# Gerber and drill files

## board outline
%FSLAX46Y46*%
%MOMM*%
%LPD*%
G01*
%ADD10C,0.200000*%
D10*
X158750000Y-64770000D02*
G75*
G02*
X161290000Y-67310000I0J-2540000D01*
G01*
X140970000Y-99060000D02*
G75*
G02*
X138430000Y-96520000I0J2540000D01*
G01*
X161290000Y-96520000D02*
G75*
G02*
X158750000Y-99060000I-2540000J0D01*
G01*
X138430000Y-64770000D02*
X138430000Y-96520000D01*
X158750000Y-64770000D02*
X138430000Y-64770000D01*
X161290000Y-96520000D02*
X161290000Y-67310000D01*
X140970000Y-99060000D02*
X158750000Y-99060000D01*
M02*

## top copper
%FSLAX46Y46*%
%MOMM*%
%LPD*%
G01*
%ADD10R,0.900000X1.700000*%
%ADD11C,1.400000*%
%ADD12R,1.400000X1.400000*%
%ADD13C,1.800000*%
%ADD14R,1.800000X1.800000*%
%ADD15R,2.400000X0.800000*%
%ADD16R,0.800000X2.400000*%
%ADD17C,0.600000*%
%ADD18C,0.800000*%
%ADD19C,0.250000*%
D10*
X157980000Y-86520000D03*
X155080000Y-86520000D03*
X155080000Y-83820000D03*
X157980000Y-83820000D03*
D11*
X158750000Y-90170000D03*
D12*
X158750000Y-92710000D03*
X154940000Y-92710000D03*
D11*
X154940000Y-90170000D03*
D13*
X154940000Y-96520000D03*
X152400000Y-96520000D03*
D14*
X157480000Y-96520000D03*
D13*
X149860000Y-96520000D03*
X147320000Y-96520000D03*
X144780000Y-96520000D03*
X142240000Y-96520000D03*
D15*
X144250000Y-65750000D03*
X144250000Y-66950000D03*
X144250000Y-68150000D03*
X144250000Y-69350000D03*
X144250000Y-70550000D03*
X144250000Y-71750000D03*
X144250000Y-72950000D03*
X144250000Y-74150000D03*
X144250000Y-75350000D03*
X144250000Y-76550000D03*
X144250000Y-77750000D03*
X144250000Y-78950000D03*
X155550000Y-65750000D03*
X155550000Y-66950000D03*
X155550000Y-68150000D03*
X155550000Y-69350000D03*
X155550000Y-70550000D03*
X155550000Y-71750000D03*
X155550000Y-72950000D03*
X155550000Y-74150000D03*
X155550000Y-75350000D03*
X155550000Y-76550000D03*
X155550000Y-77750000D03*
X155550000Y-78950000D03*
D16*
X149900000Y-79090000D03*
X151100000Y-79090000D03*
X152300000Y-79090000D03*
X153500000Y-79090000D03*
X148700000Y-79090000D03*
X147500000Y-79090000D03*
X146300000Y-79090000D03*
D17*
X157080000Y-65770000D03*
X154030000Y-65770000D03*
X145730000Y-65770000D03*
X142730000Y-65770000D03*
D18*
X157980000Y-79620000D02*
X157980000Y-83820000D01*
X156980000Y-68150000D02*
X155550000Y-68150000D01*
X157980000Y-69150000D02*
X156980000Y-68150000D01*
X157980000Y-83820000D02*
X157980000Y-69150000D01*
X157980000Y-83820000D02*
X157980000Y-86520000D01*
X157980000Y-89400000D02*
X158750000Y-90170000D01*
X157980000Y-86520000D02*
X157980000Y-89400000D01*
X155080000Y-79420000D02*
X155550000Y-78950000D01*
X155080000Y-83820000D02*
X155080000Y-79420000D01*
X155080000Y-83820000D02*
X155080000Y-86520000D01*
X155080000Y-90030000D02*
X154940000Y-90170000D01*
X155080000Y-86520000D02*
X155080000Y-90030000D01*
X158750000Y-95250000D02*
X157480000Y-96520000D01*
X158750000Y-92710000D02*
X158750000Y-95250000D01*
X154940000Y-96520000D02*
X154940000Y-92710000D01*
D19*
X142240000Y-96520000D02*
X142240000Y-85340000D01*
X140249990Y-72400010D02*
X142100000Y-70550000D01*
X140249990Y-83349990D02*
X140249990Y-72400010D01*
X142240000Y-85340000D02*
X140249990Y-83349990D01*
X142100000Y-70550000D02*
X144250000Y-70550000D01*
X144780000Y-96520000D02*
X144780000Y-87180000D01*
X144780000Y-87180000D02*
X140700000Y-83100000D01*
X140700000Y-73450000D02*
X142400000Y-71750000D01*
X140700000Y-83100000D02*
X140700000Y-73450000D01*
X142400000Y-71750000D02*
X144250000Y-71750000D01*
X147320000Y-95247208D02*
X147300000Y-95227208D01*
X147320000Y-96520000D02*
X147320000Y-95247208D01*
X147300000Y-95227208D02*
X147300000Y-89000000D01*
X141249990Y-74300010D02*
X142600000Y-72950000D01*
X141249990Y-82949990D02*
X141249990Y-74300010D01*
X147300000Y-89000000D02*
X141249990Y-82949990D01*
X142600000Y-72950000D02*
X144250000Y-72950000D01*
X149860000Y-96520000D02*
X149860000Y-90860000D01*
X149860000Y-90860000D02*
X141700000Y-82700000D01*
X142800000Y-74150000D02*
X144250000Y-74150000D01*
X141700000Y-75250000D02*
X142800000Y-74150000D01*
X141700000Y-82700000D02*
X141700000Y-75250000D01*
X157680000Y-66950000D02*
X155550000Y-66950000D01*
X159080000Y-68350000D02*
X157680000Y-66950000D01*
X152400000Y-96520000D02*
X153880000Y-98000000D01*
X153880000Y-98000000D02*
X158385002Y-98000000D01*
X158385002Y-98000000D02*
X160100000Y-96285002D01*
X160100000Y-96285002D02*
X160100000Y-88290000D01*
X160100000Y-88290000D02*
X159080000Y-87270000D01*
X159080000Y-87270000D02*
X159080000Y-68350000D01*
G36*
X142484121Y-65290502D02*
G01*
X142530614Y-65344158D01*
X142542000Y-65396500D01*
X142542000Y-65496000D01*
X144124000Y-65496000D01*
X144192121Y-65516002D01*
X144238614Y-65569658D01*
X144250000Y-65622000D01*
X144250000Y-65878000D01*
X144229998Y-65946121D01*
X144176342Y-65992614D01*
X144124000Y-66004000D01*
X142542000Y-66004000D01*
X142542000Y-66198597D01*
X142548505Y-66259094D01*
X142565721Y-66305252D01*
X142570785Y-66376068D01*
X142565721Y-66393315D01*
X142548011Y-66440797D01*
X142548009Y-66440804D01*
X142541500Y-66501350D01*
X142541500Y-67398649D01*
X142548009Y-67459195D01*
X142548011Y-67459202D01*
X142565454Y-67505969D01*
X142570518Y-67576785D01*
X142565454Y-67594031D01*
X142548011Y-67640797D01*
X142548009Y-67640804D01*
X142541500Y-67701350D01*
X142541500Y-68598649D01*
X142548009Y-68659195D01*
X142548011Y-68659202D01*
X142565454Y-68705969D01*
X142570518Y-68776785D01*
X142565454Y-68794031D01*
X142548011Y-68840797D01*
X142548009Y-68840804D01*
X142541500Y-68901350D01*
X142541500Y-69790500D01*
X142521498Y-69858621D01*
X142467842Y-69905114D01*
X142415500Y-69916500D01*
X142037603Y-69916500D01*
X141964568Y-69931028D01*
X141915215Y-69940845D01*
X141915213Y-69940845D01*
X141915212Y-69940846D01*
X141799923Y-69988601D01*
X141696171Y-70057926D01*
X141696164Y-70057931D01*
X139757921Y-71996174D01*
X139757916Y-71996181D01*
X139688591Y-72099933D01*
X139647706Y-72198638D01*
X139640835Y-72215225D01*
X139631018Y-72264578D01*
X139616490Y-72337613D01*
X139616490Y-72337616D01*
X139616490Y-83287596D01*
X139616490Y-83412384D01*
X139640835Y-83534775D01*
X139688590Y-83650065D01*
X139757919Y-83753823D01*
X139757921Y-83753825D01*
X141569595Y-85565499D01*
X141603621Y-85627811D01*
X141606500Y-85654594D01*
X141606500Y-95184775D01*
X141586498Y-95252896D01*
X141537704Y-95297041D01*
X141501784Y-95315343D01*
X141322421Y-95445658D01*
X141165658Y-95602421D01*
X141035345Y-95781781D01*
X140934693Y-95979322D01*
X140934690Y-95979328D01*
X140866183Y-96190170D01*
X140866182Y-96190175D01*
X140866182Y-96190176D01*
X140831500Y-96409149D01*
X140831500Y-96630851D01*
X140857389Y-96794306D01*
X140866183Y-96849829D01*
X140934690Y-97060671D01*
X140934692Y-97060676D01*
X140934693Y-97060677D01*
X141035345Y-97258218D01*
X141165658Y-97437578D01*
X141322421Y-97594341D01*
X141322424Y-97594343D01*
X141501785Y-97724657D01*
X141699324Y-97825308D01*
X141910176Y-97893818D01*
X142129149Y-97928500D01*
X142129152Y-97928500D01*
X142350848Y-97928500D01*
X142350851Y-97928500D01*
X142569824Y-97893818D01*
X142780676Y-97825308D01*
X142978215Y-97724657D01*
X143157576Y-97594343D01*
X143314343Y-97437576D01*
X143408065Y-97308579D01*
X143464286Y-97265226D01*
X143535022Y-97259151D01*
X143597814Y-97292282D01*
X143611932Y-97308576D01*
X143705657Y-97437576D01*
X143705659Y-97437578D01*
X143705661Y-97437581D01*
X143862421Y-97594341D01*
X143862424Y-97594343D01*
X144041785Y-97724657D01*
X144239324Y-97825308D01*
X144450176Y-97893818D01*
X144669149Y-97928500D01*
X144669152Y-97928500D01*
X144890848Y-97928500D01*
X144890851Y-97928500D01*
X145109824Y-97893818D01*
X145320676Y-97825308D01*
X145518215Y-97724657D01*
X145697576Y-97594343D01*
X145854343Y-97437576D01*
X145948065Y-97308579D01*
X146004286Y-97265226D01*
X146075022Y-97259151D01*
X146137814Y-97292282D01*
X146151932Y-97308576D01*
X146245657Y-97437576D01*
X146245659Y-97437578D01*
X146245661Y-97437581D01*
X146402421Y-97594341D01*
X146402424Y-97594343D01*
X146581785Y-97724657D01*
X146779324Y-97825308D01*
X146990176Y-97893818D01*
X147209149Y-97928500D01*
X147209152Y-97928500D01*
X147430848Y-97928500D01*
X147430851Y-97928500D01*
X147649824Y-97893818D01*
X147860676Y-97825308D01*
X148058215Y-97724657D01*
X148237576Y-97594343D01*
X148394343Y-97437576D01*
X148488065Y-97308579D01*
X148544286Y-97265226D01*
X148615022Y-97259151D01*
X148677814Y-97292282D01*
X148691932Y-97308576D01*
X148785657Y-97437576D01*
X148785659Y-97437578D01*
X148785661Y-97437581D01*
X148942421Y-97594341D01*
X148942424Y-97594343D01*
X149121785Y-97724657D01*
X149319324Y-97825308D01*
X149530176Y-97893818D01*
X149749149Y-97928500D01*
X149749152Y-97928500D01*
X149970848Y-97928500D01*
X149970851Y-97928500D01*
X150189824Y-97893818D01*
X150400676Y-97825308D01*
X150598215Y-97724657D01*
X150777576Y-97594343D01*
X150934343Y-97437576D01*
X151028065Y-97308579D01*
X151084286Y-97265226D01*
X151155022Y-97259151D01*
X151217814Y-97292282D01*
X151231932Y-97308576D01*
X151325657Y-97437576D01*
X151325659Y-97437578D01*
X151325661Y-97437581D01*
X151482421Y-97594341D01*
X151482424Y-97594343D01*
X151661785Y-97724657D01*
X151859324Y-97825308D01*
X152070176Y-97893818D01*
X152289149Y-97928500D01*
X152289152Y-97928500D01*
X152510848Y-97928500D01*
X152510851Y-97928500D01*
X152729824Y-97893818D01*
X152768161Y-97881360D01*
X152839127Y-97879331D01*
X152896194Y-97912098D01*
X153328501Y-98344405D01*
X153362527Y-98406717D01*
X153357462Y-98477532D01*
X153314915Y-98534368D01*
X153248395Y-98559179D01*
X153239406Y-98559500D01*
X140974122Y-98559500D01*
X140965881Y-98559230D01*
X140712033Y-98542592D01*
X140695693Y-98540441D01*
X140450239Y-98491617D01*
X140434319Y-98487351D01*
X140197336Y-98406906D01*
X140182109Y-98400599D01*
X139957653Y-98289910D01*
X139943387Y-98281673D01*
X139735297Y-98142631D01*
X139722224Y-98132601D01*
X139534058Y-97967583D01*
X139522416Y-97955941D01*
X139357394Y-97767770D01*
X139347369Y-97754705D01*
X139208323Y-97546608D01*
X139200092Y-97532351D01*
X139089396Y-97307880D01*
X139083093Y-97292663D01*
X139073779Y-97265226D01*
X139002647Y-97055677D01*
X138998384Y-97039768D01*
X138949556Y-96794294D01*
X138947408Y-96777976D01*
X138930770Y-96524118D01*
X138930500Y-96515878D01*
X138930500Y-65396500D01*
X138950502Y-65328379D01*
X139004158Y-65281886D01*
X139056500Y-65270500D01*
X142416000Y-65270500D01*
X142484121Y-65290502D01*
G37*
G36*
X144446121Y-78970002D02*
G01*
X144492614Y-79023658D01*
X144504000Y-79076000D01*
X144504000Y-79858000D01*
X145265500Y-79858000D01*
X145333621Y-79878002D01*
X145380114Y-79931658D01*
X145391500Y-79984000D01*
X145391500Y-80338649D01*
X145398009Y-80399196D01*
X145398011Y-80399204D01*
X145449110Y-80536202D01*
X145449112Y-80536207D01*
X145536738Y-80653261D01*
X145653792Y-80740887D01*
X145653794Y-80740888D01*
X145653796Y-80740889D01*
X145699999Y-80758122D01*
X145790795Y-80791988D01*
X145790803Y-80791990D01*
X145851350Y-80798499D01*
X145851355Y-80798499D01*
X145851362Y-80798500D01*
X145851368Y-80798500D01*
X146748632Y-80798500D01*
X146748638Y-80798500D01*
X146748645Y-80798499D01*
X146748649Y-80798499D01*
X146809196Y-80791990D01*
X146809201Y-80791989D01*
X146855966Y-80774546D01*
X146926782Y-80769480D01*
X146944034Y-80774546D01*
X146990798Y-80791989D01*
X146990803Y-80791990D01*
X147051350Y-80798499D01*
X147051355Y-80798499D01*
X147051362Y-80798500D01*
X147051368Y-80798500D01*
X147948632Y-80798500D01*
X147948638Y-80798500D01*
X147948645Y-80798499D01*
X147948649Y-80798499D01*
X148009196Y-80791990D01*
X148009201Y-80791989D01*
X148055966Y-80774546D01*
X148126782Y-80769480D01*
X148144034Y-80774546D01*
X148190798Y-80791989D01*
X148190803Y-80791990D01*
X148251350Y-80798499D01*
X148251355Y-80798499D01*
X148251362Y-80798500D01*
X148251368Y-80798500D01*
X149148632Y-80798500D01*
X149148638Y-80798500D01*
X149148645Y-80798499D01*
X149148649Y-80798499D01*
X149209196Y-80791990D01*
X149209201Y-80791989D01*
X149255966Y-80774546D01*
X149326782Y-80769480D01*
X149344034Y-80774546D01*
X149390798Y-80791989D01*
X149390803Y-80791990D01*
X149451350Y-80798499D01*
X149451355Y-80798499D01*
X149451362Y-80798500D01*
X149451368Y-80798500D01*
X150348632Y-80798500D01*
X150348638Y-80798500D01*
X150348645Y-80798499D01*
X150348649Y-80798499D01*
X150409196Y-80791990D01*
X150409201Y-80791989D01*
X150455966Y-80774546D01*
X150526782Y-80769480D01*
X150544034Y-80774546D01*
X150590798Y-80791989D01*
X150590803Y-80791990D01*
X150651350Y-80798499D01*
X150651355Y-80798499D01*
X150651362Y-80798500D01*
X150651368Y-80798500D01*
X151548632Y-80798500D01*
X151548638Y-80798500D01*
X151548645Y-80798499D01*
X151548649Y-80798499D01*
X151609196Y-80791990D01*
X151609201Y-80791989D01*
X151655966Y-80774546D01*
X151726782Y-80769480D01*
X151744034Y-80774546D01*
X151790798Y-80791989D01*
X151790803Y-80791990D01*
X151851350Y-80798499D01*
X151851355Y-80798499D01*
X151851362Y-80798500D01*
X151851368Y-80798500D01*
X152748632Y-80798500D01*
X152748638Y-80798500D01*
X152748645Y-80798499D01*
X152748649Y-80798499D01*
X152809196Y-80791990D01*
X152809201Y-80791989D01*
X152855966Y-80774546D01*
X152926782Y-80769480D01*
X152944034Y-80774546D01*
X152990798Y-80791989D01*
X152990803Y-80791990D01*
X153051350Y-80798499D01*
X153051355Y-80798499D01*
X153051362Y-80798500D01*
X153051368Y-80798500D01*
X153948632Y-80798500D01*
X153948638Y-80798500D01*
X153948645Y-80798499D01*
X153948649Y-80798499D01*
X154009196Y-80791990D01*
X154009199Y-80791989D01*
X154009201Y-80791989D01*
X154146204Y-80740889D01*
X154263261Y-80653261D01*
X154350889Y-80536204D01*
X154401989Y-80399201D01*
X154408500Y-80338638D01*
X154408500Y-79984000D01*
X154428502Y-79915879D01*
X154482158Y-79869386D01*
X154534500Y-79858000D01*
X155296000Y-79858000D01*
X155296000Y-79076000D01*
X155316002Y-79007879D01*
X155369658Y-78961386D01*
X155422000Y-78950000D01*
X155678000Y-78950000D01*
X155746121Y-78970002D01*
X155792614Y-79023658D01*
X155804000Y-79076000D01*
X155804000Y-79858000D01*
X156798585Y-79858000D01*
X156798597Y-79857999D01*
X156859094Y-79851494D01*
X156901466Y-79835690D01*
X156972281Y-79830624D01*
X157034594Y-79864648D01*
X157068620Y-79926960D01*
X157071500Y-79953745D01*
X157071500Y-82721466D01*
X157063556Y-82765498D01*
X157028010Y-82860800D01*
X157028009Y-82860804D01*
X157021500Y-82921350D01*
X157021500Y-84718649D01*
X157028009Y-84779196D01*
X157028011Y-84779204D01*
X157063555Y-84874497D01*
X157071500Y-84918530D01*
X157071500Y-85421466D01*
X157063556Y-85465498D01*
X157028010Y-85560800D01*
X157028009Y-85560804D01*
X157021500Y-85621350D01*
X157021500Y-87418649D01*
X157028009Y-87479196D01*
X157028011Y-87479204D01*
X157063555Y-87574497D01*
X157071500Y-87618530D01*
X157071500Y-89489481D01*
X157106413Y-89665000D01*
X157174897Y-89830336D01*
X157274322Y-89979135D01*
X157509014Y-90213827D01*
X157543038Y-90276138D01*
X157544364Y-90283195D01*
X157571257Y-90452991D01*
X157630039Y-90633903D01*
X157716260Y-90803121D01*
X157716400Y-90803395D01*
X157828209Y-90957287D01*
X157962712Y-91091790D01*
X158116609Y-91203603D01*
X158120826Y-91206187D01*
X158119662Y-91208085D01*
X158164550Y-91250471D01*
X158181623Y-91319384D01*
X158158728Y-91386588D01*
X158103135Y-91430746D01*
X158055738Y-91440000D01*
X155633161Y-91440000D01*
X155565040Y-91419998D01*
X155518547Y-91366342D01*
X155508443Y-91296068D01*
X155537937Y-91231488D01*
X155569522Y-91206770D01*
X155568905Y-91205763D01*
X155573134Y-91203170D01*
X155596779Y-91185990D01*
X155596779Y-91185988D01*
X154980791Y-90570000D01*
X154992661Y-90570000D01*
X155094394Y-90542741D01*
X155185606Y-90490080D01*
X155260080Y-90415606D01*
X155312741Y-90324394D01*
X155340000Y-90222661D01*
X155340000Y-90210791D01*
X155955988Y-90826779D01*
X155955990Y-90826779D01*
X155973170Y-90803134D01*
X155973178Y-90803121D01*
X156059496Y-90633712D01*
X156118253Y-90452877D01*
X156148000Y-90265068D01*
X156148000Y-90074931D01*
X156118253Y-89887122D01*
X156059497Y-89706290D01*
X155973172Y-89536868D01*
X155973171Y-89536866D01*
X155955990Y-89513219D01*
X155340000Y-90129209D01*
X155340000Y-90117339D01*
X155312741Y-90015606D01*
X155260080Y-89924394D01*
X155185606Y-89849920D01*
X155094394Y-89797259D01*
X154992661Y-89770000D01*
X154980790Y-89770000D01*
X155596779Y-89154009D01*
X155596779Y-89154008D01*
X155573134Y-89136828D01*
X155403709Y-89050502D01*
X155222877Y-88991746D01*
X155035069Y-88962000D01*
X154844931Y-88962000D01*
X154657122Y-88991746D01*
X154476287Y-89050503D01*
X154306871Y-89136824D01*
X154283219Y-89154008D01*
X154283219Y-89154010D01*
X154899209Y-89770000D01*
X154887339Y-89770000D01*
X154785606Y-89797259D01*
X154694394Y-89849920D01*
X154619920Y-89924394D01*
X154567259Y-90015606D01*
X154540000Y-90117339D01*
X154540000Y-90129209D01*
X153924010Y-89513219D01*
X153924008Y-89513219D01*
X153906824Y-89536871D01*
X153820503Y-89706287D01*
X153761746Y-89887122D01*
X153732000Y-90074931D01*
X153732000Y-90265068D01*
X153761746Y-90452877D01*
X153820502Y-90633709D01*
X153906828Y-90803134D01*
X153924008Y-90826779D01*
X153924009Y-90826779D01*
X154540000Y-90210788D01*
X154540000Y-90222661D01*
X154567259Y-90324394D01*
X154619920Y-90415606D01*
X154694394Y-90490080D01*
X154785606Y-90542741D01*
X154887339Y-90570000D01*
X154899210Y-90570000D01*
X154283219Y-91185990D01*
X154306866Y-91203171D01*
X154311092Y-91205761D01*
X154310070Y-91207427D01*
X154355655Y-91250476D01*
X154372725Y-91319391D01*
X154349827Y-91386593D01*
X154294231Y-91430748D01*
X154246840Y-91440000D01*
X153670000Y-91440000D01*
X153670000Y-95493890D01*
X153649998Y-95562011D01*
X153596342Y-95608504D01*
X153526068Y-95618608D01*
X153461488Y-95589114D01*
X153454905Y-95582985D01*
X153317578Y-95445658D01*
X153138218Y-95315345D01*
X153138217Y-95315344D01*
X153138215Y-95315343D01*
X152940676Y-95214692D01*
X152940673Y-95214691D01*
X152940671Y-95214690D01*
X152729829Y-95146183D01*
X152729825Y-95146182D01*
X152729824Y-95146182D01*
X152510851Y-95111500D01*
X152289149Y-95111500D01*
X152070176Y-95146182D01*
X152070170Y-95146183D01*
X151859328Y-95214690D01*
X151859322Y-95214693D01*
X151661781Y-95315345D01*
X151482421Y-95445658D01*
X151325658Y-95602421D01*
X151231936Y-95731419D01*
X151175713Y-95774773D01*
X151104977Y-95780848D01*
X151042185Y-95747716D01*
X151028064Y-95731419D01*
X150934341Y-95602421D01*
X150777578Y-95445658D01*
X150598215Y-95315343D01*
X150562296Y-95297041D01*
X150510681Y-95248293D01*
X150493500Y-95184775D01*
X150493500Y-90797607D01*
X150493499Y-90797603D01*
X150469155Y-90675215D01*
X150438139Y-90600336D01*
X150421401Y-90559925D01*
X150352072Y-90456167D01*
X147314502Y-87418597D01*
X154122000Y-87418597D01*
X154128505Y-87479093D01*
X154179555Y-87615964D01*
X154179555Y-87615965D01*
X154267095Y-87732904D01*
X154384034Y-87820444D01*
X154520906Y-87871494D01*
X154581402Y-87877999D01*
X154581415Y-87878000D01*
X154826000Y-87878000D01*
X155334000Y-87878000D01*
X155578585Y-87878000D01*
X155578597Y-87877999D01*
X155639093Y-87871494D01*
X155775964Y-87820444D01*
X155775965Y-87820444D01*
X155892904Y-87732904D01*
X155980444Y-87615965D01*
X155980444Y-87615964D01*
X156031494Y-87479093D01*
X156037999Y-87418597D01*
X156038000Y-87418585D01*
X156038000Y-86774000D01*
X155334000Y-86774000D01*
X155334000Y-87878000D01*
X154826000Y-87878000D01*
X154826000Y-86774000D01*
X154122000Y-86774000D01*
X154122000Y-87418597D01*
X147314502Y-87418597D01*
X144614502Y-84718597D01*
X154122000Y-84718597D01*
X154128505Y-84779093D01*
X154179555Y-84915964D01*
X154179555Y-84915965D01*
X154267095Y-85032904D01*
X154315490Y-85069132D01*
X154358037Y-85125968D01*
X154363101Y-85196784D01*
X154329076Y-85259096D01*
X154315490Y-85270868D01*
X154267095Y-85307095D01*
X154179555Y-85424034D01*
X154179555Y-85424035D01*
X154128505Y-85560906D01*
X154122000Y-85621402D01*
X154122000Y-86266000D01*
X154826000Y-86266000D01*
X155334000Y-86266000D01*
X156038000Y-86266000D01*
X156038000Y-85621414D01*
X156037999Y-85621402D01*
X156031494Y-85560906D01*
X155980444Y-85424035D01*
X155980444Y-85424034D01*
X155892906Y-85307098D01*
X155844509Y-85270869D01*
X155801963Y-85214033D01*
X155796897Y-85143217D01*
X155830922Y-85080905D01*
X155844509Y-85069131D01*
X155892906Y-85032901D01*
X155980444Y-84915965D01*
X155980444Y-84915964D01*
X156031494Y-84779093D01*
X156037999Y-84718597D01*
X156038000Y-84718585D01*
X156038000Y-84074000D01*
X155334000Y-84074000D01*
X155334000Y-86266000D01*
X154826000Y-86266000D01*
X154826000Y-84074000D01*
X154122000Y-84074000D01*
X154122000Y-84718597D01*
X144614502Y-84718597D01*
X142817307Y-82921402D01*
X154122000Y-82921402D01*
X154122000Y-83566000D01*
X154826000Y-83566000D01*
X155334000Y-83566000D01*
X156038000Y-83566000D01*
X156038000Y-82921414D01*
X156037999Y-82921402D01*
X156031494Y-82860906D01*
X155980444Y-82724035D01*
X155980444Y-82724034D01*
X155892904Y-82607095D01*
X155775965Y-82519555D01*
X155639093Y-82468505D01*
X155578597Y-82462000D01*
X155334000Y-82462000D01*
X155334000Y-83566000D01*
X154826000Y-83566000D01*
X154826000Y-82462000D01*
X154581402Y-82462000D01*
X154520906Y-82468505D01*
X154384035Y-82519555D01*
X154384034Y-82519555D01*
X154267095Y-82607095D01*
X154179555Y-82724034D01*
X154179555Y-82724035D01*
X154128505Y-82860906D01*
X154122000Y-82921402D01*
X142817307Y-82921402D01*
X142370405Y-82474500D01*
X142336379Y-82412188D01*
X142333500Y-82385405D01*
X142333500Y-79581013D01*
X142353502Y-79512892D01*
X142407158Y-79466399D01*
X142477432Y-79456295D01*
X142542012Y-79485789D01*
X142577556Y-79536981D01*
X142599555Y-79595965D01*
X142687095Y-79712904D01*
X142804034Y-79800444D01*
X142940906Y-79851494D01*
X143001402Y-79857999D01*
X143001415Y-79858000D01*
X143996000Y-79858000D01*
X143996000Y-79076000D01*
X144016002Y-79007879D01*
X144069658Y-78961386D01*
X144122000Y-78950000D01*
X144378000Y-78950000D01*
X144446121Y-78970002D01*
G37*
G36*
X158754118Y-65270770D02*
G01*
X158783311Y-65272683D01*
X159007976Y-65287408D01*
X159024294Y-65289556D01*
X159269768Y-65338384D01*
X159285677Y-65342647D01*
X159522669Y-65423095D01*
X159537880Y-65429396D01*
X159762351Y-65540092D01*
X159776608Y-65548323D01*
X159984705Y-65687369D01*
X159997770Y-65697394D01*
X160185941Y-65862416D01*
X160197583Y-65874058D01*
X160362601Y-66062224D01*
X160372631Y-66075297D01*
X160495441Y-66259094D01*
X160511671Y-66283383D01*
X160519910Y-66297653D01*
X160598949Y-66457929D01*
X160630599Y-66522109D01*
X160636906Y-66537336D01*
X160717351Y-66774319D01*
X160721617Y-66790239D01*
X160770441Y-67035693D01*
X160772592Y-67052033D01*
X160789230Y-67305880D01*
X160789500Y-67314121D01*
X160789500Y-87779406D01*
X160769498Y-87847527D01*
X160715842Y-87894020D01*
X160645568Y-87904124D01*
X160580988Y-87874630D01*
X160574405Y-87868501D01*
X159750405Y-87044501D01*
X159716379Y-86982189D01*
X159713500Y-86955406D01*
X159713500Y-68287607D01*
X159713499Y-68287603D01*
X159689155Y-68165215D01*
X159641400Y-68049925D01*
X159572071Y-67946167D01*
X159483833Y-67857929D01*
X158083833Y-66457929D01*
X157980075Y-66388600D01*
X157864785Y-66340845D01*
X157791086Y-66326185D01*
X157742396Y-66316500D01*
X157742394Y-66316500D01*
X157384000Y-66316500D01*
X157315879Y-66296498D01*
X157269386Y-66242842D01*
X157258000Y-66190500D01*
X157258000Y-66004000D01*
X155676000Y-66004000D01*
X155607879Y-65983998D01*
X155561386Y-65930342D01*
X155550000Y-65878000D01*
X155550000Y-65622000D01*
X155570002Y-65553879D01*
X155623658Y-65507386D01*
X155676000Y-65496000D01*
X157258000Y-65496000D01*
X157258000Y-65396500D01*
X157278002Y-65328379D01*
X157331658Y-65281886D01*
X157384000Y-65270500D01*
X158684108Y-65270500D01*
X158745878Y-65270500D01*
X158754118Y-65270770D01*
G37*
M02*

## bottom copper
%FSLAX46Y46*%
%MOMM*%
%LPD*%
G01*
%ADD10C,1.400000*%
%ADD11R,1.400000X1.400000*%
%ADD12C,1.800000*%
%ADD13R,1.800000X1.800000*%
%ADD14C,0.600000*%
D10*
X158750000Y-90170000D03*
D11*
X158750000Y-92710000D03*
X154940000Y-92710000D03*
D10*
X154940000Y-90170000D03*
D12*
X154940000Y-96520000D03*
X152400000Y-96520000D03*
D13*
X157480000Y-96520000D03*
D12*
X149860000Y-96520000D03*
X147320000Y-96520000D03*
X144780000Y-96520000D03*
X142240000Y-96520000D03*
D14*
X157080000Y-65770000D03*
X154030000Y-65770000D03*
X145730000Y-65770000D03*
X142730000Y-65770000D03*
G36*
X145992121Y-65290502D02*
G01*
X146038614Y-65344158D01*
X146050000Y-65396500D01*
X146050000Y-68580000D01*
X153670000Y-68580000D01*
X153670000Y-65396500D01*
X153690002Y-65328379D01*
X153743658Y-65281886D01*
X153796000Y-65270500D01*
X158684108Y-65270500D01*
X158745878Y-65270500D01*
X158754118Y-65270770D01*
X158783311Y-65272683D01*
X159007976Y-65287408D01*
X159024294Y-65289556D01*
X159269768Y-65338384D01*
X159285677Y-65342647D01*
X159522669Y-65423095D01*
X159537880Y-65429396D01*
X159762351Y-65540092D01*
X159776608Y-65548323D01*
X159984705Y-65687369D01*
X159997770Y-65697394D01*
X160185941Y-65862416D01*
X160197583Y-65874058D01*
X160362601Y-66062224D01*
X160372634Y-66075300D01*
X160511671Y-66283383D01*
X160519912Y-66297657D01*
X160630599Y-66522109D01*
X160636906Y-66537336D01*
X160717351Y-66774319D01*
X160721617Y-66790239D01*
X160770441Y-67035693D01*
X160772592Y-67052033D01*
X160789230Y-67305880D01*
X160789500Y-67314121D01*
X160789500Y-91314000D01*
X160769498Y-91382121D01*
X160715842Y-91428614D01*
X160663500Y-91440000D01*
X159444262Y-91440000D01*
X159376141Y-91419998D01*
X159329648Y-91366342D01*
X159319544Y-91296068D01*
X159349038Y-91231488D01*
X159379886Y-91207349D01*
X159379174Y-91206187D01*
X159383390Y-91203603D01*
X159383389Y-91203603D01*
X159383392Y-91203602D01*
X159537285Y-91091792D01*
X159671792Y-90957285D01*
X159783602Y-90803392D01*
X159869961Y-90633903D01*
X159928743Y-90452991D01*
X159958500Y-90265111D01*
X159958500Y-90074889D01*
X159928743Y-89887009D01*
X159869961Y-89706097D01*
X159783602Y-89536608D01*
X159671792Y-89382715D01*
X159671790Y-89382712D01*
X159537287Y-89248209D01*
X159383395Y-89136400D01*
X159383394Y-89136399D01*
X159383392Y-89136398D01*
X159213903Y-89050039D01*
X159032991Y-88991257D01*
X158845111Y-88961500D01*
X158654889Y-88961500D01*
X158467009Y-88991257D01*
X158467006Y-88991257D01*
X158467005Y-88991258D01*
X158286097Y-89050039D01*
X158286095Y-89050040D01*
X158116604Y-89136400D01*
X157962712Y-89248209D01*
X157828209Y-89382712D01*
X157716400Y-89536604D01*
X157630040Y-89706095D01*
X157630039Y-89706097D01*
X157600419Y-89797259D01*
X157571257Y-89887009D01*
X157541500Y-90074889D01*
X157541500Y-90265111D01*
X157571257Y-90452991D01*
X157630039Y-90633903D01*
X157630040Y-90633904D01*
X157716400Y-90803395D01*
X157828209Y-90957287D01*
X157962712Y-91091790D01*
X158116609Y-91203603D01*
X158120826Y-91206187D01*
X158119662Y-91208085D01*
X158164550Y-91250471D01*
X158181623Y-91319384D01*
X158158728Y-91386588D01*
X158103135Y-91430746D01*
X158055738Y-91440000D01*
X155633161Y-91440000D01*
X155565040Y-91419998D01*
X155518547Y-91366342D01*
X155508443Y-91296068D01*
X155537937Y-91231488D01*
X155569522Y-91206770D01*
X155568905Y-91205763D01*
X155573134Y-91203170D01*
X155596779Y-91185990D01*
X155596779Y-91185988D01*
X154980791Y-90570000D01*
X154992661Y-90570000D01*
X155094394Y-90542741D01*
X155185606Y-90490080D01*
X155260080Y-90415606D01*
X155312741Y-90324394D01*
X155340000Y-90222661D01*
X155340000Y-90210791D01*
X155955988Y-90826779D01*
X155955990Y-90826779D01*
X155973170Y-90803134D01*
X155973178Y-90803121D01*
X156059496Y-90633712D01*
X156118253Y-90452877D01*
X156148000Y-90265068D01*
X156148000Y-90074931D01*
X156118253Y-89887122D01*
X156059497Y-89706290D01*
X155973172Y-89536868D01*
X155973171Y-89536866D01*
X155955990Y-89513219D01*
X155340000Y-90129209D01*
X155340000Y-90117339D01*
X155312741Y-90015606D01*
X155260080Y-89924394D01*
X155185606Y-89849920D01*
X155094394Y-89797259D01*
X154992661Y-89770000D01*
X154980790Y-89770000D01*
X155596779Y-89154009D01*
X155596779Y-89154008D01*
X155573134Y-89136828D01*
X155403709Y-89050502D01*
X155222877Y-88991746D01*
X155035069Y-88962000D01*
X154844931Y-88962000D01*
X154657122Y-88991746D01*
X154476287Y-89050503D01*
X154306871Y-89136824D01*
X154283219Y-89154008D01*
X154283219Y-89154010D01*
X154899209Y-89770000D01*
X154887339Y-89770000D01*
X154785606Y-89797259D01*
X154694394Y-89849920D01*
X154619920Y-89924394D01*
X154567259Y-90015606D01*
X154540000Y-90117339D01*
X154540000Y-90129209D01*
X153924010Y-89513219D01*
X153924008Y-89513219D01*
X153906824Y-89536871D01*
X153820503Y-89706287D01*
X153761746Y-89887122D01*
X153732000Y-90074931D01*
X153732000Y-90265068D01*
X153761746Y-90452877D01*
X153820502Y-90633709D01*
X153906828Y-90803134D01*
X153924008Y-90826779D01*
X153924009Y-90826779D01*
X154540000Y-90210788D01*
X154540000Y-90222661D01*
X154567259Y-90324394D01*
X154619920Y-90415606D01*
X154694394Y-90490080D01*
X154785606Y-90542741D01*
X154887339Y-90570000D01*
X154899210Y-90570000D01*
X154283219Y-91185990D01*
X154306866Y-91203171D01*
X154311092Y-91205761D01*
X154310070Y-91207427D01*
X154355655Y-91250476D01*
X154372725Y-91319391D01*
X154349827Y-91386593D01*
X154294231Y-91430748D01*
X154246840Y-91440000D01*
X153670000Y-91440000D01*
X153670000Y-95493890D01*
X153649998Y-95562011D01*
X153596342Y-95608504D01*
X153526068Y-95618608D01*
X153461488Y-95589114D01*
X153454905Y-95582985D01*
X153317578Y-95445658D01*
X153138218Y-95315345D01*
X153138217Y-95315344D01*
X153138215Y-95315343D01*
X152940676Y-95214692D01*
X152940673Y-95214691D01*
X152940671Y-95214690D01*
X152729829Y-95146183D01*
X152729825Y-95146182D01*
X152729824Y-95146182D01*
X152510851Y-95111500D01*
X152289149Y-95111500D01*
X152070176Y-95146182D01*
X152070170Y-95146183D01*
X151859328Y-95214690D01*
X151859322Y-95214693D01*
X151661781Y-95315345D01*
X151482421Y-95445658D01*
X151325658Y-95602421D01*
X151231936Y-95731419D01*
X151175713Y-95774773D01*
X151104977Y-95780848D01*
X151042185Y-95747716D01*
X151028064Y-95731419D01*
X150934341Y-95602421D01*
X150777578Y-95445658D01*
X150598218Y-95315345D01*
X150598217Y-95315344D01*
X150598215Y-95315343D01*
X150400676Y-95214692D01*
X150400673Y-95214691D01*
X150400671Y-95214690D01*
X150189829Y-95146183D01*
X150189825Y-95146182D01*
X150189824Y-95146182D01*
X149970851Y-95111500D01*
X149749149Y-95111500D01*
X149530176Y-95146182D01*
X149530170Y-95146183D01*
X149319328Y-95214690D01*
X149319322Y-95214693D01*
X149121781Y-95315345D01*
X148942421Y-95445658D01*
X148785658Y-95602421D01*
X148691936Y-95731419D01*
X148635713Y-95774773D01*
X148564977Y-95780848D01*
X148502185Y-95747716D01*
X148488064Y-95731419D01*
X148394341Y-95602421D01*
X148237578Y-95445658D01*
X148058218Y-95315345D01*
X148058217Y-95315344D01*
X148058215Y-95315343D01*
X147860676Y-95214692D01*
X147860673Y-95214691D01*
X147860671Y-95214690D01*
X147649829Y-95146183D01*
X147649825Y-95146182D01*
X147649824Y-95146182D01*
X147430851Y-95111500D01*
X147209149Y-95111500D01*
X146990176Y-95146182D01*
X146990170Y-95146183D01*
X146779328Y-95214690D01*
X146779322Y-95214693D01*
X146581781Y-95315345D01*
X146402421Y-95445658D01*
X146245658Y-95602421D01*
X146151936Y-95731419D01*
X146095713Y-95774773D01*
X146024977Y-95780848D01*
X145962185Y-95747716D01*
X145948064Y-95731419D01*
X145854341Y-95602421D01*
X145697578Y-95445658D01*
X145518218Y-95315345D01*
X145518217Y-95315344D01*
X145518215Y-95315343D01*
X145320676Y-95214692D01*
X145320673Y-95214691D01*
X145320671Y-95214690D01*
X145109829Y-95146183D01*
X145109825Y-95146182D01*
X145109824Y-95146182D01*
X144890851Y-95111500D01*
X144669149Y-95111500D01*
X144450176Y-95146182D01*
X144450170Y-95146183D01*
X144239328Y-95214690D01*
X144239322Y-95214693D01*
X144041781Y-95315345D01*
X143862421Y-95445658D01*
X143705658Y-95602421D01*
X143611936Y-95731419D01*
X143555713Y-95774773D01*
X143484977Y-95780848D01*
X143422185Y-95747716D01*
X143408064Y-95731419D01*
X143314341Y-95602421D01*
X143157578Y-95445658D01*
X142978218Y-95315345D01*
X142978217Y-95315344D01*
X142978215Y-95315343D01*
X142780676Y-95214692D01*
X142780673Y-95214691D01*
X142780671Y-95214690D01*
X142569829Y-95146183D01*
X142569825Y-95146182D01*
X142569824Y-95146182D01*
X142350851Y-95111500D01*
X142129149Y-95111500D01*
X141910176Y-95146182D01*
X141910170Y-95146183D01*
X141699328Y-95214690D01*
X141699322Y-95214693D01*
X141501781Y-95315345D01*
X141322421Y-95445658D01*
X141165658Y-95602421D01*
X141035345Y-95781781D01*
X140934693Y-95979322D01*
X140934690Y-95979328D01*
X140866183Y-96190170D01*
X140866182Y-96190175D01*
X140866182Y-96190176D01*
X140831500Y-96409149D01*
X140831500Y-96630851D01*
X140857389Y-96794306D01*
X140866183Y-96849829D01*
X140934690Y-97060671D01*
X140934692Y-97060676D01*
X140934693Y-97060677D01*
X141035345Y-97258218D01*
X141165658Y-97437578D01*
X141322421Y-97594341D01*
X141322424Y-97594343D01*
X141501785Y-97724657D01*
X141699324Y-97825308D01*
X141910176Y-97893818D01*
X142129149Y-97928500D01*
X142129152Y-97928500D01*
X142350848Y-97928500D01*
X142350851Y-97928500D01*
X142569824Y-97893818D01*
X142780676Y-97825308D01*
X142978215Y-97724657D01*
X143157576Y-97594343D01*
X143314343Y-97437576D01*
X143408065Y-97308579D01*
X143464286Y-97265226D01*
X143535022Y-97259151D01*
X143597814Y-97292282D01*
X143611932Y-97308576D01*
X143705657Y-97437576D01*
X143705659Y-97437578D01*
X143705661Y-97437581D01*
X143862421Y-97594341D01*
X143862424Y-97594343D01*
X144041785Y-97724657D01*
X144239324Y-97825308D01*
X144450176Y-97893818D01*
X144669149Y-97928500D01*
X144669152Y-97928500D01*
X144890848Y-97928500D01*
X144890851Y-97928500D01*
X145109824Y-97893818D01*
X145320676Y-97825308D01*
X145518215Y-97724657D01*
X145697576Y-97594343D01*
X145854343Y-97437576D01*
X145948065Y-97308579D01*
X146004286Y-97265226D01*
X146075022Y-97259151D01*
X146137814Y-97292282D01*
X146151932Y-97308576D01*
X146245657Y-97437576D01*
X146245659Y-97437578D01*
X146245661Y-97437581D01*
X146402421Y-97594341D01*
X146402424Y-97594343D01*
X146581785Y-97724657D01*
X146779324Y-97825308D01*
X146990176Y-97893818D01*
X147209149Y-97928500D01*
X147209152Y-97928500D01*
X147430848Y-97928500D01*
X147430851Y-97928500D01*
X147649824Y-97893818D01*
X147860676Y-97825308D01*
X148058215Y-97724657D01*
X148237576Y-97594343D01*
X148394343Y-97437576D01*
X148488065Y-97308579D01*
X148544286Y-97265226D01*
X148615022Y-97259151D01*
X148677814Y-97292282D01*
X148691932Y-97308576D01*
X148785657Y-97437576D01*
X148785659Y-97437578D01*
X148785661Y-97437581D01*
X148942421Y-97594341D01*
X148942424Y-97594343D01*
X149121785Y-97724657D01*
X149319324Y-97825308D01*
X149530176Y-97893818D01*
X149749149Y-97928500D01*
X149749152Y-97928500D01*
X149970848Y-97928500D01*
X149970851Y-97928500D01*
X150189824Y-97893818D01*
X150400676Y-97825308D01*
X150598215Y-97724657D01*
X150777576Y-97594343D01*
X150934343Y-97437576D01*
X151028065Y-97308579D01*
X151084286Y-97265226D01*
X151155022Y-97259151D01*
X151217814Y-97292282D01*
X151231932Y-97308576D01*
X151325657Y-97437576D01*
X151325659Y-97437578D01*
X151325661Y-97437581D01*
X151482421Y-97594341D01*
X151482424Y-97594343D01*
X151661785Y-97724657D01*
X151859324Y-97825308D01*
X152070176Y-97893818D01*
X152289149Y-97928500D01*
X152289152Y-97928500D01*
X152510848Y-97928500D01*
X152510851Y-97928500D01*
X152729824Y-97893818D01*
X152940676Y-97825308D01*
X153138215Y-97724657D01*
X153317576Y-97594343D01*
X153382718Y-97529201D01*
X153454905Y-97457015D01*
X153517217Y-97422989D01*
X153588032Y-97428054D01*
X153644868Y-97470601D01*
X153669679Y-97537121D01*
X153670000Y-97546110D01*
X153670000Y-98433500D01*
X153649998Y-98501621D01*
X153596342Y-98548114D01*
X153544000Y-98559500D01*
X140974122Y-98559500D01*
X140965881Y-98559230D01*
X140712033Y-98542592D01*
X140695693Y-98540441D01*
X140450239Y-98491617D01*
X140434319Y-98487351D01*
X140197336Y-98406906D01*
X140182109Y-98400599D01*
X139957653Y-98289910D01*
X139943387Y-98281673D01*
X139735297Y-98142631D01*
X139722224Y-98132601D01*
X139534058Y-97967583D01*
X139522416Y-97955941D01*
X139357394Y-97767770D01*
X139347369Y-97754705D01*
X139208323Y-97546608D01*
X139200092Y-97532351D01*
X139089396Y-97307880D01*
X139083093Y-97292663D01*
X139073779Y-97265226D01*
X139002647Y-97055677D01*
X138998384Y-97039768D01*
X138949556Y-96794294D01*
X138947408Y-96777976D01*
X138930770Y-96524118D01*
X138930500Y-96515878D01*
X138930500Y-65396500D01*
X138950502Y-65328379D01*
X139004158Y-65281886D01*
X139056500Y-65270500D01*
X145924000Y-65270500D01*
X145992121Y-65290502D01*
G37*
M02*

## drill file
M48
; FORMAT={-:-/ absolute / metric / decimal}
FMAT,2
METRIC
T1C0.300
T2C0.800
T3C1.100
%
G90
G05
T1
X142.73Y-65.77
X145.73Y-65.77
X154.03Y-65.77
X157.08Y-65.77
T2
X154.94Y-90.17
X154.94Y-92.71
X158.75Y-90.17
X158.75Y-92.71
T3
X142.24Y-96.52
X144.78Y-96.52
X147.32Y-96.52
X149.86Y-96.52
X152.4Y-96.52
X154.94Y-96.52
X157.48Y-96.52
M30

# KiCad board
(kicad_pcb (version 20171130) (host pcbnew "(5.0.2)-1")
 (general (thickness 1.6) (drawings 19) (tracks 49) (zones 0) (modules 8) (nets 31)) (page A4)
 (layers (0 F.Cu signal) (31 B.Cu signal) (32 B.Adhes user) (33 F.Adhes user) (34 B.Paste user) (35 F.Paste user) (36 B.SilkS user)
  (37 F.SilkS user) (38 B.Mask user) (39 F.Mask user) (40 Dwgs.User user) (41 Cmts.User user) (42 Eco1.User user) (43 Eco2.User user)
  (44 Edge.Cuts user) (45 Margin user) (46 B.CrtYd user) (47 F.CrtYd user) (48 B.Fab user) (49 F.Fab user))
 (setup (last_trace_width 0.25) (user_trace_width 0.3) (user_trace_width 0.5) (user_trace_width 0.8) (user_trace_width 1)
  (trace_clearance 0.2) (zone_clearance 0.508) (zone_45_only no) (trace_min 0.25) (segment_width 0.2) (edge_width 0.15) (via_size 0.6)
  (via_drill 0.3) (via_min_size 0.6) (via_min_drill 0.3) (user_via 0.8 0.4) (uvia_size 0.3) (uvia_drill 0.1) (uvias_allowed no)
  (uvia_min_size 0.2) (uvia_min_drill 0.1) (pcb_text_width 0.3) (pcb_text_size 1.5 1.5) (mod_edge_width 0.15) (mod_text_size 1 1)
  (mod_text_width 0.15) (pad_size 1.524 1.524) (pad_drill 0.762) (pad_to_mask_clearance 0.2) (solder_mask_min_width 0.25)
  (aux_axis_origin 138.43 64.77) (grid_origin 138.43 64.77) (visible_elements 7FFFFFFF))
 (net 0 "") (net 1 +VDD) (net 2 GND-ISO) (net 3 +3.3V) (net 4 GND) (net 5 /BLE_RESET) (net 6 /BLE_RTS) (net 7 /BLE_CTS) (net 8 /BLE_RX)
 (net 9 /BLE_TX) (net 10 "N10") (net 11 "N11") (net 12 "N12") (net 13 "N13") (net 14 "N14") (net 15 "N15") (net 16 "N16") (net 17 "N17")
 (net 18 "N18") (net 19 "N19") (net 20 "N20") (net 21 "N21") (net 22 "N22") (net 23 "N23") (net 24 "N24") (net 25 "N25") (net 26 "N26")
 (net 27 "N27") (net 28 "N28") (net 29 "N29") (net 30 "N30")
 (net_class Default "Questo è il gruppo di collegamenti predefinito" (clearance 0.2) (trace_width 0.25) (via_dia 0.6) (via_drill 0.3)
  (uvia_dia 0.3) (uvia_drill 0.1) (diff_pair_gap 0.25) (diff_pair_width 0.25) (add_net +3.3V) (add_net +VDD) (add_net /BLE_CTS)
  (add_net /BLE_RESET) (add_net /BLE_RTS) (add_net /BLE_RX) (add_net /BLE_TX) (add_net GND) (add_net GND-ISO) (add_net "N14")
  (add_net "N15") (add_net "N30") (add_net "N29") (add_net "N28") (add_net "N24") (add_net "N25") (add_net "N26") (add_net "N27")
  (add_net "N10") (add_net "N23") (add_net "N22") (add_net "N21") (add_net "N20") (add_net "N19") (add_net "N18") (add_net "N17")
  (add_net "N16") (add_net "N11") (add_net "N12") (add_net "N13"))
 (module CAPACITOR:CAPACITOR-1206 (layer F.Cu) (at 156.53 86.52 180)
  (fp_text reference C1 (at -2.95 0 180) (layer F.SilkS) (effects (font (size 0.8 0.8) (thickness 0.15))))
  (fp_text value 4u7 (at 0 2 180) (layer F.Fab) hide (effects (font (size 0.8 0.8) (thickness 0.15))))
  (pad 1 smd rect (at -1.45 0 180) (size 0.9 1.7) (layers F.Cu F.Paste F.Mask) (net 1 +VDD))
  (pad 2 smd rect (at 1.45 0 180) (size 0.9 1.7) (layers F.Cu F.Paste F.Mask) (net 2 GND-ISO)))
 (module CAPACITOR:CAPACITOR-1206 (layer F.Cu) (at 156.53 83.82 180)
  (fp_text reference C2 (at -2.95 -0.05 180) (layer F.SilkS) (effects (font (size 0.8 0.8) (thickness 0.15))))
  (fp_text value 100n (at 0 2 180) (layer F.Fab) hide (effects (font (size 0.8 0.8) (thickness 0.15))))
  (pad 2 smd rect (at 1.45 0 180) (size 0.9 1.7) (layers F.Cu F.Paste F.Mask) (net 2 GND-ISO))
  (pad 1 smd rect (at -1.45 0 180) (size 0.9 1.7) (layers F.Cu F.Paste F.Mask) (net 1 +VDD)))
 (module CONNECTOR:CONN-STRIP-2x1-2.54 (layer F.Cu) (at 158.75 91.44 90)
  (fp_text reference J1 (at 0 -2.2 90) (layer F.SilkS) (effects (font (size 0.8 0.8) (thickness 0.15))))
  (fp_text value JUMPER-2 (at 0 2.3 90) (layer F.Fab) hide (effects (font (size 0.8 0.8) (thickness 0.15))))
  (pad 2 thru_hole circle (at 1.27 0 90) (size 1.4 1.4) (drill 0.8) (layers *.Cu *.Mask) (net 1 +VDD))
  (pad 1 thru_hole rect (at -1.27 0 90) (size 1.4 1.4) (drill 0.8) (layers *.Cu *.Mask) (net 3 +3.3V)))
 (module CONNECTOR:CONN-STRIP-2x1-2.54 (layer F.Cu) (at 154.94 91.44 90)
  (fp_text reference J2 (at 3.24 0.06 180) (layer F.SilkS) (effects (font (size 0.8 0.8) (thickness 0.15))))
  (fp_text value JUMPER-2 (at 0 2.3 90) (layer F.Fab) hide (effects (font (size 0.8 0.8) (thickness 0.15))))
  (pad 1 thru_hole rect (at -1.27 0 90) (size 1.4 1.4) (drill 0.8) (layers *.Cu *.Mask) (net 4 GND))
  (pad 2 thru_hole circle (at 1.27 0 90) (size 1.4 1.4) (drill 0.8) (layers *.Cu *.Mask) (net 2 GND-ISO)))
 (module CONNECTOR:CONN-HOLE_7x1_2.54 (layer F.Cu) (at 149.86 96.52 180)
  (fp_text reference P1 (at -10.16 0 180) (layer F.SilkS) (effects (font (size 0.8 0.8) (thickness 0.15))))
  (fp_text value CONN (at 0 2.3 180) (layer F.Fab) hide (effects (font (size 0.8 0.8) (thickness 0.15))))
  (pad 2 thru_hole circle (at -5.08 0 180) (size 1.8 1.8) (drill 1.1) (layers *.Cu *.Mask) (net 4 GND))
  (pad 3 thru_hole circle (at -2.54 0 180) (size 1.8 1.8) (drill 1.1) (layers *.Cu *.Mask) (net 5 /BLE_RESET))
  (pad 1 thru_hole rect (at -7.62 0 180) (size 1.8 1.8) (drill 1.1) (layers *.Cu *.Mask) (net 3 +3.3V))
  (pad 4 thru_hole circle (at 0 0 180) (size 1.8 1.8) (drill 1.1) (layers *.Cu *.Mask) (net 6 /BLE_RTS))
  (pad 5 thru_hole circle (at 2.54 0 180) (size 1.8 1.8) (drill 1.1) (layers *.Cu *.Mask) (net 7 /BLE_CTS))
  (pad 6 thru_hole circle (at 5.08 0 180) (size 1.8 1.8) (drill 1.1) (layers *.Cu *.Mask) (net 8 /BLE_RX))
  (pad 7 thru_hole circle (at 7.62 0 180) (size 1.8 1.8) (drill 1.1) (layers *.Cu *.Mask) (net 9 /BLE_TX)))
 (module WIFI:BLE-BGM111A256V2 (layer F.Cu) (at 149.9 72.39)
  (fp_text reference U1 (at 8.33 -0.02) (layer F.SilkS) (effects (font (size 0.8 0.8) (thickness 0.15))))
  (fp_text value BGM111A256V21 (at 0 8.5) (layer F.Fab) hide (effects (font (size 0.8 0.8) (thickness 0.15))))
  (pad 1 smd rect (at -5.65 -6.64) (size 2.4 0.8) (layers F.Cu F.Paste F.Mask) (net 2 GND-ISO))
  (pad 2 smd rect (at -5.65 -5.44) (size 2.4 0.8) (layers F.Cu F.Paste F.Mask) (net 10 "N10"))
  (pad 3 smd rect (at -5.65 -4.24) (size 2.4 0.8) (layers F.Cu F.Paste F.Mask) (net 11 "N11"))
  (pad 4 smd rect (at -5.65 -3.04) (size 2.4 0.8) (layers F.Cu F.Paste F.Mask) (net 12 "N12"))
  (pad 5 smd rect (at -5.65 -1.84) (size 2.4 0.8) (layers F.Cu F.Paste F.Mask) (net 9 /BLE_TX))
  (pad 6 smd rect (at -5.65 -0.64) (size 2.4 0.8) (layers F.Cu F.Paste F.Mask) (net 8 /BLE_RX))
  (pad 7 smd rect (at -5.65 0.56) (size 2.4 0.8) (layers F.Cu F.Paste F.Mask) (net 7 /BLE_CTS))
  (pad 8 smd rect (at -5.65 1.76) (size 2.4 0.8) (layers F.Cu F.Paste F.Mask) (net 6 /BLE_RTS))
  (pad 9 smd rect (at -5.65 2.96) (size 2.4 0.8) (layers F.Cu F.Paste F.Mask) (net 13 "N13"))
  (pad 10 smd rect (at -5.65 4.16) (size 2.4 0.8) (layers F.Cu F.Paste F.Mask) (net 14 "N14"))
  (pad 11 smd rect (at -5.65 5.36) (size 2.4 0.8) (layers F.Cu F.Paste F.Mask) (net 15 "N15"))
  (pad 12 smd rect (at -5.65 6.56) (size 2.4 0.8) (layers F.Cu F.Paste F.Mask) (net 2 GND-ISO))
  (pad 31 smd rect (at 5.65 -6.64) (size 2.4 0.8) (layers F.Cu F.Paste F.Mask) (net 2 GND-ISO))
  (pad 30 smd rect (at 5.65 -5.44) (size 2.4 0.8) (layers F.Cu F.Paste F.Mask) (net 5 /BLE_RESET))
  (pad 29 smd rect (at 5.65 -4.24) (size 2.4 0.8) (layers F.Cu F.Paste F.Mask) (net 1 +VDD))
  (pad 28 smd rect (at 5.65 -3.04) (size 2.4 0.8) (layers F.Cu F.Paste F.Mask) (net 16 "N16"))
  (pad 27 smd rect (at 5.65 -1.84) (size 2.4 0.8) (layers F.Cu F.Paste F.Mask) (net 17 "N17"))
  (pad 26 smd rect (at 5.65 -0.64) (size 2.4 0.8) (layers F.Cu F.Paste F.Mask) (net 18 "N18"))
  (pad 25 smd rect (at 5.65 0.56) (size 2.4 0.8) (layers F.Cu F.Paste F.Mask) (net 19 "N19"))
  (pad 24 smd rect (at 5.65 1.76) (size 2.4 0.8) (layers F.Cu F.Paste F.Mask) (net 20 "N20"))
  (pad 23 smd rect (at 5.65 2.96) (size 2.4 0.8) (layers F.Cu F.Paste F.Mask) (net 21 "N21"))
  (pad 22 smd rect (at 5.65 4.16) (size 2.4 0.8) (layers F.Cu F.Paste F.Mask) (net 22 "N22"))
  (pad 21 smd rect (at 5.65 5.36) (size 2.4 0.8) (layers F.Cu F.Paste F.Mask) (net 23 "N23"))
  (pad 20 smd rect (at 5.65 6.56) (size 2.4 0.8) (layers F.Cu F.Paste F.Mask) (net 2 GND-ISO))
  (pad 16 smd rect (at 0 6.7 90) (size 2.4 0.8) (layers F.Cu F.Paste F.Mask) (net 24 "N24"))
  (pad 17 smd rect (at 1.2 6.7 90) (size 2.4 0.8) (layers F.Cu F.Paste F.Mask) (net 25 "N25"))
  (pad 18 smd rect (at 2.4 6.7 90) (size 2.4 0.8) (layers F.Cu F.Paste F.Mask) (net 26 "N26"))
  (pad 19 smd rect (at 3.6 6.7 90) (size 2.4 0.8) (layers F.Cu F.Paste F.Mask) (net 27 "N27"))
  (pad 15 smd rect (at -1.2 6.7 90) (size 2.4 0.8) (layers F.Cu F.Paste F.Mask) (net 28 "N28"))
  (pad 14 smd rect (at -2.4 6.7 90) (size 2.4 0.8) (layers F.Cu F.Paste F.Mask) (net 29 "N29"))
  (pad 13 smd rect (at -3.6 6.7 90) (size 2.4 0.8) (layers F.Cu F.Paste F.Mask) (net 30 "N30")))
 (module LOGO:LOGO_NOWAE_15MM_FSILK (layer F.Cu) (at 147.2 83.5)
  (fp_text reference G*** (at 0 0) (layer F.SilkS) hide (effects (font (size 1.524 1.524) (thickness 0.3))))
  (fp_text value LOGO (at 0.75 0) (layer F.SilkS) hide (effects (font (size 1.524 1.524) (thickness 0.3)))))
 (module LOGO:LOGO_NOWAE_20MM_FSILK (layer B.Cu) (at 149.86 78.74 180)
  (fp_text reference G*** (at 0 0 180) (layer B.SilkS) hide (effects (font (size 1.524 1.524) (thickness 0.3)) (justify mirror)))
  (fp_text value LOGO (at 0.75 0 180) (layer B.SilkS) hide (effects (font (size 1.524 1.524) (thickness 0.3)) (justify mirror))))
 (gr_arc (start 158.75 67.31) (end 161.29 67.31) (angle -90) (layer Edge.Cuts) (width 0.2))
 (gr_arc (start 140.97 96.52) (end 138.43 96.52) (angle -90) (layer Edge.Cuts) (width 0.2))
 (gr_arc (start 158.75 96.52) (end 158.75 99.06) (angle -90) (layer Edge.Cuts) (width 0.2))
 (gr_line (start 138.43 64.77) (end 138.43 96.52) (layer Edge.Cuts) (width 0.2))
 (gr_line (start 158.75 64.77) (end 138.43 64.77) (layer Edge.Cuts) (width 0.2))
 (gr_line (start 161.29 96.52) (end 161.29 67.31) (layer Edge.Cuts) (width 0.2))
 (gr_line (start 140.97 99.06) (end 158.75 99.06) (layer Edge.Cuts) (width 0.2))
 (segment (start 157.98 79.62) (end 157.98 83.82) (width 0.8) (layer F.Cu) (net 1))
 (segment (start 156.98 68.15) (end 155.55 68.15) (width 0.8) (layer F.Cu) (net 1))
 (segment (start 157.98 69.15) (end 156.98 68.15) (width 0.8) (layer F.Cu) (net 1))
 (segment (start 157.98 83.82) (end 157.98 69.15) (width 0.8) (layer F.Cu) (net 1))
 (segment (start 157.98 83.82) (end 157.98 86.52) (width 0.8) (layer F.Cu) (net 1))
 (segment (start 157.98 89.4) (end 158.75 90.17) (width 0.8) (layer F.Cu) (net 1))
 (segment (start 157.98 86.52) (end 157.98 89.4) (width 0.8) (layer F.Cu) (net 1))
 (via (at 157.08 65.77) (size 0.6) (drill 0.3) (layers F.Cu B.Cu) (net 2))
 (via (at 154.03 65.77) (size 0.6) (drill 0.3) (layers F.Cu B.Cu) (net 2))
 (via (at 145.73 65.77) (size 0.6) (drill 0.3) (layers F.Cu B.Cu) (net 2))
 (via (at 142.73 65.77) (size 0.6) (drill 0.3) (layers F.Cu B.Cu) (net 2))
 (segment (start 155.08 79.42) (end 155.55 78.95) (width 0.8) (layer F.Cu) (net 2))
 (segment (start 155.08 83.82) (end 155.08 79.42) (width 0.8) (layer F.Cu) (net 2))
 (segment (start 155.08 83.82) (end 155.08 86.52) (width 0.8) (layer F.Cu) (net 2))
 (segment (start 155.08 90.03) (end 154.94 90.17) (width 0.8) (layer F.Cu) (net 2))
 (segment (start 155.08 86.52) (end 155.08 90.03) (width 0.8) (layer F.Cu) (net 2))
 (segment (start 158.75 95.25) (end 157.48 96.52) (width 0.8) (layer F.Cu) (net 3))
 (segment (start 158.75 92.71) (end 158.75 95.25) (width 0.8) (layer F.Cu) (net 3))
 (segment (start 154.94 96.52) (end 154.94 92.71) (width 0.8) (layer F.Cu) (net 4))
 (segment (start 142.24 96.52) (end 142.24 85.34) (width 0.25) (layer F.Cu) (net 9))
 (segment (start 140.24999 72.40001) (end 142.1 70.55) (width 0.25) (layer F.Cu) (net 9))
 (segment (start 140.24999 83.34999) (end 140.24999 72.40001) (width 0.25) (layer F.Cu) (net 9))
 (segment (start 142.24 85.34) (end 140.24999 83.34999) (width 0.25) (layer F.Cu) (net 9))
 (segment (start 142.1 70.55) (end 144.25 70.55) (width 0.25) (layer F.Cu) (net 9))
 (segment (start 144.78 96.52) (end 144.78 87.18) (width 0.25) (layer F.Cu) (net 8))
 (segment (start 144.78 87.18) (end 140.7 83.1) (width 0.25) (layer F.Cu) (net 8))
 (segment (start 140.7 73.45) (end 142.4 71.75) (width 0.25) (layer F.Cu) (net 8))
 (segment (start 140.7 83.1) (end 140.7 73.45) (width 0.25) (layer F.Cu) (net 8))
 (segment (start 142.4 71.75) (end 144.25 71.75) (width 0.25) (layer F.Cu) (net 8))
 (segment (start 147.32 95.247208) (end 147.3 95.227208) (width 0.25) (layer F.Cu) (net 7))
 (segment (start 147.32 96.52) (end 147.32 95.247208) (width 0.25) (layer F.Cu) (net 7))
 (segment (start 147.3 95.227208) (end 147.3 89) (width 0.25) (layer F.Cu) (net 7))
 (segment (start 141.24999 74.30001) (end 142.6 72.95) (width 0.25) (layer F.Cu) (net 7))
 (segment (start 141.24999 82.94999) (end 141.24999 74.30001) (width 0.25) (layer F.Cu) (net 7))
 (segment (start 147.3 89) (end 141.24999 82.94999) (width 0.25) (layer F.Cu) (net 7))
 (segment (start 142.6 72.95) (end 144.25 72.95) (width 0.25) (layer F.Cu) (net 7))
 (segment (start 149.86 96.52) (end 149.86 90.86) (width 0.25) (layer F.Cu) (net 6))
 (segment (start 149.86 90.86) (end 141.7 82.7) (width 0.25) (layer F.Cu) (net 6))
 (segment (start 142.8 74.15) (end 144.25 74.15) (width 0.25) (layer F.Cu) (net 6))
 (segment (start 141.7 75.25) (end 142.8 74.15) (width 0.25) (layer F.Cu) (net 6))
 (segment (start 141.7 82.7) (end 141.7 75.25) (width 0.25) (layer F.Cu) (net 6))
 (segment (start 157.68 66.95) (end 155.55 66.95) (width 0.25) (layer F.Cu) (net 5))
 (segment (start 159.08 68.35) (end 157.68 66.95) (width 0.25) (layer F.Cu) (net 5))
 (segment (start 152.4 96.52) (end 153.88 98) (width 0.25) (layer F.Cu) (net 5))
 (segment (start 153.88 98) (end 158.385002 98) (width 0.25) (layer F.Cu) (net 5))
 (segment (start 158.385002 98) (end 160.1 96.285002) (width 0.25) (layer F.Cu) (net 5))
 (segment (start 160.1 96.285002) (end 160.1 88.29) (width 0.25) (layer F.Cu) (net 5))
 (segment (start 160.1 88.29) (end 159.08 87.27) (width 0.25) (layer F.Cu) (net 5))
 (segment (start 159.08 87.27) (end 159.08 68.35) (width 0.25) (layer F.Cu) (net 5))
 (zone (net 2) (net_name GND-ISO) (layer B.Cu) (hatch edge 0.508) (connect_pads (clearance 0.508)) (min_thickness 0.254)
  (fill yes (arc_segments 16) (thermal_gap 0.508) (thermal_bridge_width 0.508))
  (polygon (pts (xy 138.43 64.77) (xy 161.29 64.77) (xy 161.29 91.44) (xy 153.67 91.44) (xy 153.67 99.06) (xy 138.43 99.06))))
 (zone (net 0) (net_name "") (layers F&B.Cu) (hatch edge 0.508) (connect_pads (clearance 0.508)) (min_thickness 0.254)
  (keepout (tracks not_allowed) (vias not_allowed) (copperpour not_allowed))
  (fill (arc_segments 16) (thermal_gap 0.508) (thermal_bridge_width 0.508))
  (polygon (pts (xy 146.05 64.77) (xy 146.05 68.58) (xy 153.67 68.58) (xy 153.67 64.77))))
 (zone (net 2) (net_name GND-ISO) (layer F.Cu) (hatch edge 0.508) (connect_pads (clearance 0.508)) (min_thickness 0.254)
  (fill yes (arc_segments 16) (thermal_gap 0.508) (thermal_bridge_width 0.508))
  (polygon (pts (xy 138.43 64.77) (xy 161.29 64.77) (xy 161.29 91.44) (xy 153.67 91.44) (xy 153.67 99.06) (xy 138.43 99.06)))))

